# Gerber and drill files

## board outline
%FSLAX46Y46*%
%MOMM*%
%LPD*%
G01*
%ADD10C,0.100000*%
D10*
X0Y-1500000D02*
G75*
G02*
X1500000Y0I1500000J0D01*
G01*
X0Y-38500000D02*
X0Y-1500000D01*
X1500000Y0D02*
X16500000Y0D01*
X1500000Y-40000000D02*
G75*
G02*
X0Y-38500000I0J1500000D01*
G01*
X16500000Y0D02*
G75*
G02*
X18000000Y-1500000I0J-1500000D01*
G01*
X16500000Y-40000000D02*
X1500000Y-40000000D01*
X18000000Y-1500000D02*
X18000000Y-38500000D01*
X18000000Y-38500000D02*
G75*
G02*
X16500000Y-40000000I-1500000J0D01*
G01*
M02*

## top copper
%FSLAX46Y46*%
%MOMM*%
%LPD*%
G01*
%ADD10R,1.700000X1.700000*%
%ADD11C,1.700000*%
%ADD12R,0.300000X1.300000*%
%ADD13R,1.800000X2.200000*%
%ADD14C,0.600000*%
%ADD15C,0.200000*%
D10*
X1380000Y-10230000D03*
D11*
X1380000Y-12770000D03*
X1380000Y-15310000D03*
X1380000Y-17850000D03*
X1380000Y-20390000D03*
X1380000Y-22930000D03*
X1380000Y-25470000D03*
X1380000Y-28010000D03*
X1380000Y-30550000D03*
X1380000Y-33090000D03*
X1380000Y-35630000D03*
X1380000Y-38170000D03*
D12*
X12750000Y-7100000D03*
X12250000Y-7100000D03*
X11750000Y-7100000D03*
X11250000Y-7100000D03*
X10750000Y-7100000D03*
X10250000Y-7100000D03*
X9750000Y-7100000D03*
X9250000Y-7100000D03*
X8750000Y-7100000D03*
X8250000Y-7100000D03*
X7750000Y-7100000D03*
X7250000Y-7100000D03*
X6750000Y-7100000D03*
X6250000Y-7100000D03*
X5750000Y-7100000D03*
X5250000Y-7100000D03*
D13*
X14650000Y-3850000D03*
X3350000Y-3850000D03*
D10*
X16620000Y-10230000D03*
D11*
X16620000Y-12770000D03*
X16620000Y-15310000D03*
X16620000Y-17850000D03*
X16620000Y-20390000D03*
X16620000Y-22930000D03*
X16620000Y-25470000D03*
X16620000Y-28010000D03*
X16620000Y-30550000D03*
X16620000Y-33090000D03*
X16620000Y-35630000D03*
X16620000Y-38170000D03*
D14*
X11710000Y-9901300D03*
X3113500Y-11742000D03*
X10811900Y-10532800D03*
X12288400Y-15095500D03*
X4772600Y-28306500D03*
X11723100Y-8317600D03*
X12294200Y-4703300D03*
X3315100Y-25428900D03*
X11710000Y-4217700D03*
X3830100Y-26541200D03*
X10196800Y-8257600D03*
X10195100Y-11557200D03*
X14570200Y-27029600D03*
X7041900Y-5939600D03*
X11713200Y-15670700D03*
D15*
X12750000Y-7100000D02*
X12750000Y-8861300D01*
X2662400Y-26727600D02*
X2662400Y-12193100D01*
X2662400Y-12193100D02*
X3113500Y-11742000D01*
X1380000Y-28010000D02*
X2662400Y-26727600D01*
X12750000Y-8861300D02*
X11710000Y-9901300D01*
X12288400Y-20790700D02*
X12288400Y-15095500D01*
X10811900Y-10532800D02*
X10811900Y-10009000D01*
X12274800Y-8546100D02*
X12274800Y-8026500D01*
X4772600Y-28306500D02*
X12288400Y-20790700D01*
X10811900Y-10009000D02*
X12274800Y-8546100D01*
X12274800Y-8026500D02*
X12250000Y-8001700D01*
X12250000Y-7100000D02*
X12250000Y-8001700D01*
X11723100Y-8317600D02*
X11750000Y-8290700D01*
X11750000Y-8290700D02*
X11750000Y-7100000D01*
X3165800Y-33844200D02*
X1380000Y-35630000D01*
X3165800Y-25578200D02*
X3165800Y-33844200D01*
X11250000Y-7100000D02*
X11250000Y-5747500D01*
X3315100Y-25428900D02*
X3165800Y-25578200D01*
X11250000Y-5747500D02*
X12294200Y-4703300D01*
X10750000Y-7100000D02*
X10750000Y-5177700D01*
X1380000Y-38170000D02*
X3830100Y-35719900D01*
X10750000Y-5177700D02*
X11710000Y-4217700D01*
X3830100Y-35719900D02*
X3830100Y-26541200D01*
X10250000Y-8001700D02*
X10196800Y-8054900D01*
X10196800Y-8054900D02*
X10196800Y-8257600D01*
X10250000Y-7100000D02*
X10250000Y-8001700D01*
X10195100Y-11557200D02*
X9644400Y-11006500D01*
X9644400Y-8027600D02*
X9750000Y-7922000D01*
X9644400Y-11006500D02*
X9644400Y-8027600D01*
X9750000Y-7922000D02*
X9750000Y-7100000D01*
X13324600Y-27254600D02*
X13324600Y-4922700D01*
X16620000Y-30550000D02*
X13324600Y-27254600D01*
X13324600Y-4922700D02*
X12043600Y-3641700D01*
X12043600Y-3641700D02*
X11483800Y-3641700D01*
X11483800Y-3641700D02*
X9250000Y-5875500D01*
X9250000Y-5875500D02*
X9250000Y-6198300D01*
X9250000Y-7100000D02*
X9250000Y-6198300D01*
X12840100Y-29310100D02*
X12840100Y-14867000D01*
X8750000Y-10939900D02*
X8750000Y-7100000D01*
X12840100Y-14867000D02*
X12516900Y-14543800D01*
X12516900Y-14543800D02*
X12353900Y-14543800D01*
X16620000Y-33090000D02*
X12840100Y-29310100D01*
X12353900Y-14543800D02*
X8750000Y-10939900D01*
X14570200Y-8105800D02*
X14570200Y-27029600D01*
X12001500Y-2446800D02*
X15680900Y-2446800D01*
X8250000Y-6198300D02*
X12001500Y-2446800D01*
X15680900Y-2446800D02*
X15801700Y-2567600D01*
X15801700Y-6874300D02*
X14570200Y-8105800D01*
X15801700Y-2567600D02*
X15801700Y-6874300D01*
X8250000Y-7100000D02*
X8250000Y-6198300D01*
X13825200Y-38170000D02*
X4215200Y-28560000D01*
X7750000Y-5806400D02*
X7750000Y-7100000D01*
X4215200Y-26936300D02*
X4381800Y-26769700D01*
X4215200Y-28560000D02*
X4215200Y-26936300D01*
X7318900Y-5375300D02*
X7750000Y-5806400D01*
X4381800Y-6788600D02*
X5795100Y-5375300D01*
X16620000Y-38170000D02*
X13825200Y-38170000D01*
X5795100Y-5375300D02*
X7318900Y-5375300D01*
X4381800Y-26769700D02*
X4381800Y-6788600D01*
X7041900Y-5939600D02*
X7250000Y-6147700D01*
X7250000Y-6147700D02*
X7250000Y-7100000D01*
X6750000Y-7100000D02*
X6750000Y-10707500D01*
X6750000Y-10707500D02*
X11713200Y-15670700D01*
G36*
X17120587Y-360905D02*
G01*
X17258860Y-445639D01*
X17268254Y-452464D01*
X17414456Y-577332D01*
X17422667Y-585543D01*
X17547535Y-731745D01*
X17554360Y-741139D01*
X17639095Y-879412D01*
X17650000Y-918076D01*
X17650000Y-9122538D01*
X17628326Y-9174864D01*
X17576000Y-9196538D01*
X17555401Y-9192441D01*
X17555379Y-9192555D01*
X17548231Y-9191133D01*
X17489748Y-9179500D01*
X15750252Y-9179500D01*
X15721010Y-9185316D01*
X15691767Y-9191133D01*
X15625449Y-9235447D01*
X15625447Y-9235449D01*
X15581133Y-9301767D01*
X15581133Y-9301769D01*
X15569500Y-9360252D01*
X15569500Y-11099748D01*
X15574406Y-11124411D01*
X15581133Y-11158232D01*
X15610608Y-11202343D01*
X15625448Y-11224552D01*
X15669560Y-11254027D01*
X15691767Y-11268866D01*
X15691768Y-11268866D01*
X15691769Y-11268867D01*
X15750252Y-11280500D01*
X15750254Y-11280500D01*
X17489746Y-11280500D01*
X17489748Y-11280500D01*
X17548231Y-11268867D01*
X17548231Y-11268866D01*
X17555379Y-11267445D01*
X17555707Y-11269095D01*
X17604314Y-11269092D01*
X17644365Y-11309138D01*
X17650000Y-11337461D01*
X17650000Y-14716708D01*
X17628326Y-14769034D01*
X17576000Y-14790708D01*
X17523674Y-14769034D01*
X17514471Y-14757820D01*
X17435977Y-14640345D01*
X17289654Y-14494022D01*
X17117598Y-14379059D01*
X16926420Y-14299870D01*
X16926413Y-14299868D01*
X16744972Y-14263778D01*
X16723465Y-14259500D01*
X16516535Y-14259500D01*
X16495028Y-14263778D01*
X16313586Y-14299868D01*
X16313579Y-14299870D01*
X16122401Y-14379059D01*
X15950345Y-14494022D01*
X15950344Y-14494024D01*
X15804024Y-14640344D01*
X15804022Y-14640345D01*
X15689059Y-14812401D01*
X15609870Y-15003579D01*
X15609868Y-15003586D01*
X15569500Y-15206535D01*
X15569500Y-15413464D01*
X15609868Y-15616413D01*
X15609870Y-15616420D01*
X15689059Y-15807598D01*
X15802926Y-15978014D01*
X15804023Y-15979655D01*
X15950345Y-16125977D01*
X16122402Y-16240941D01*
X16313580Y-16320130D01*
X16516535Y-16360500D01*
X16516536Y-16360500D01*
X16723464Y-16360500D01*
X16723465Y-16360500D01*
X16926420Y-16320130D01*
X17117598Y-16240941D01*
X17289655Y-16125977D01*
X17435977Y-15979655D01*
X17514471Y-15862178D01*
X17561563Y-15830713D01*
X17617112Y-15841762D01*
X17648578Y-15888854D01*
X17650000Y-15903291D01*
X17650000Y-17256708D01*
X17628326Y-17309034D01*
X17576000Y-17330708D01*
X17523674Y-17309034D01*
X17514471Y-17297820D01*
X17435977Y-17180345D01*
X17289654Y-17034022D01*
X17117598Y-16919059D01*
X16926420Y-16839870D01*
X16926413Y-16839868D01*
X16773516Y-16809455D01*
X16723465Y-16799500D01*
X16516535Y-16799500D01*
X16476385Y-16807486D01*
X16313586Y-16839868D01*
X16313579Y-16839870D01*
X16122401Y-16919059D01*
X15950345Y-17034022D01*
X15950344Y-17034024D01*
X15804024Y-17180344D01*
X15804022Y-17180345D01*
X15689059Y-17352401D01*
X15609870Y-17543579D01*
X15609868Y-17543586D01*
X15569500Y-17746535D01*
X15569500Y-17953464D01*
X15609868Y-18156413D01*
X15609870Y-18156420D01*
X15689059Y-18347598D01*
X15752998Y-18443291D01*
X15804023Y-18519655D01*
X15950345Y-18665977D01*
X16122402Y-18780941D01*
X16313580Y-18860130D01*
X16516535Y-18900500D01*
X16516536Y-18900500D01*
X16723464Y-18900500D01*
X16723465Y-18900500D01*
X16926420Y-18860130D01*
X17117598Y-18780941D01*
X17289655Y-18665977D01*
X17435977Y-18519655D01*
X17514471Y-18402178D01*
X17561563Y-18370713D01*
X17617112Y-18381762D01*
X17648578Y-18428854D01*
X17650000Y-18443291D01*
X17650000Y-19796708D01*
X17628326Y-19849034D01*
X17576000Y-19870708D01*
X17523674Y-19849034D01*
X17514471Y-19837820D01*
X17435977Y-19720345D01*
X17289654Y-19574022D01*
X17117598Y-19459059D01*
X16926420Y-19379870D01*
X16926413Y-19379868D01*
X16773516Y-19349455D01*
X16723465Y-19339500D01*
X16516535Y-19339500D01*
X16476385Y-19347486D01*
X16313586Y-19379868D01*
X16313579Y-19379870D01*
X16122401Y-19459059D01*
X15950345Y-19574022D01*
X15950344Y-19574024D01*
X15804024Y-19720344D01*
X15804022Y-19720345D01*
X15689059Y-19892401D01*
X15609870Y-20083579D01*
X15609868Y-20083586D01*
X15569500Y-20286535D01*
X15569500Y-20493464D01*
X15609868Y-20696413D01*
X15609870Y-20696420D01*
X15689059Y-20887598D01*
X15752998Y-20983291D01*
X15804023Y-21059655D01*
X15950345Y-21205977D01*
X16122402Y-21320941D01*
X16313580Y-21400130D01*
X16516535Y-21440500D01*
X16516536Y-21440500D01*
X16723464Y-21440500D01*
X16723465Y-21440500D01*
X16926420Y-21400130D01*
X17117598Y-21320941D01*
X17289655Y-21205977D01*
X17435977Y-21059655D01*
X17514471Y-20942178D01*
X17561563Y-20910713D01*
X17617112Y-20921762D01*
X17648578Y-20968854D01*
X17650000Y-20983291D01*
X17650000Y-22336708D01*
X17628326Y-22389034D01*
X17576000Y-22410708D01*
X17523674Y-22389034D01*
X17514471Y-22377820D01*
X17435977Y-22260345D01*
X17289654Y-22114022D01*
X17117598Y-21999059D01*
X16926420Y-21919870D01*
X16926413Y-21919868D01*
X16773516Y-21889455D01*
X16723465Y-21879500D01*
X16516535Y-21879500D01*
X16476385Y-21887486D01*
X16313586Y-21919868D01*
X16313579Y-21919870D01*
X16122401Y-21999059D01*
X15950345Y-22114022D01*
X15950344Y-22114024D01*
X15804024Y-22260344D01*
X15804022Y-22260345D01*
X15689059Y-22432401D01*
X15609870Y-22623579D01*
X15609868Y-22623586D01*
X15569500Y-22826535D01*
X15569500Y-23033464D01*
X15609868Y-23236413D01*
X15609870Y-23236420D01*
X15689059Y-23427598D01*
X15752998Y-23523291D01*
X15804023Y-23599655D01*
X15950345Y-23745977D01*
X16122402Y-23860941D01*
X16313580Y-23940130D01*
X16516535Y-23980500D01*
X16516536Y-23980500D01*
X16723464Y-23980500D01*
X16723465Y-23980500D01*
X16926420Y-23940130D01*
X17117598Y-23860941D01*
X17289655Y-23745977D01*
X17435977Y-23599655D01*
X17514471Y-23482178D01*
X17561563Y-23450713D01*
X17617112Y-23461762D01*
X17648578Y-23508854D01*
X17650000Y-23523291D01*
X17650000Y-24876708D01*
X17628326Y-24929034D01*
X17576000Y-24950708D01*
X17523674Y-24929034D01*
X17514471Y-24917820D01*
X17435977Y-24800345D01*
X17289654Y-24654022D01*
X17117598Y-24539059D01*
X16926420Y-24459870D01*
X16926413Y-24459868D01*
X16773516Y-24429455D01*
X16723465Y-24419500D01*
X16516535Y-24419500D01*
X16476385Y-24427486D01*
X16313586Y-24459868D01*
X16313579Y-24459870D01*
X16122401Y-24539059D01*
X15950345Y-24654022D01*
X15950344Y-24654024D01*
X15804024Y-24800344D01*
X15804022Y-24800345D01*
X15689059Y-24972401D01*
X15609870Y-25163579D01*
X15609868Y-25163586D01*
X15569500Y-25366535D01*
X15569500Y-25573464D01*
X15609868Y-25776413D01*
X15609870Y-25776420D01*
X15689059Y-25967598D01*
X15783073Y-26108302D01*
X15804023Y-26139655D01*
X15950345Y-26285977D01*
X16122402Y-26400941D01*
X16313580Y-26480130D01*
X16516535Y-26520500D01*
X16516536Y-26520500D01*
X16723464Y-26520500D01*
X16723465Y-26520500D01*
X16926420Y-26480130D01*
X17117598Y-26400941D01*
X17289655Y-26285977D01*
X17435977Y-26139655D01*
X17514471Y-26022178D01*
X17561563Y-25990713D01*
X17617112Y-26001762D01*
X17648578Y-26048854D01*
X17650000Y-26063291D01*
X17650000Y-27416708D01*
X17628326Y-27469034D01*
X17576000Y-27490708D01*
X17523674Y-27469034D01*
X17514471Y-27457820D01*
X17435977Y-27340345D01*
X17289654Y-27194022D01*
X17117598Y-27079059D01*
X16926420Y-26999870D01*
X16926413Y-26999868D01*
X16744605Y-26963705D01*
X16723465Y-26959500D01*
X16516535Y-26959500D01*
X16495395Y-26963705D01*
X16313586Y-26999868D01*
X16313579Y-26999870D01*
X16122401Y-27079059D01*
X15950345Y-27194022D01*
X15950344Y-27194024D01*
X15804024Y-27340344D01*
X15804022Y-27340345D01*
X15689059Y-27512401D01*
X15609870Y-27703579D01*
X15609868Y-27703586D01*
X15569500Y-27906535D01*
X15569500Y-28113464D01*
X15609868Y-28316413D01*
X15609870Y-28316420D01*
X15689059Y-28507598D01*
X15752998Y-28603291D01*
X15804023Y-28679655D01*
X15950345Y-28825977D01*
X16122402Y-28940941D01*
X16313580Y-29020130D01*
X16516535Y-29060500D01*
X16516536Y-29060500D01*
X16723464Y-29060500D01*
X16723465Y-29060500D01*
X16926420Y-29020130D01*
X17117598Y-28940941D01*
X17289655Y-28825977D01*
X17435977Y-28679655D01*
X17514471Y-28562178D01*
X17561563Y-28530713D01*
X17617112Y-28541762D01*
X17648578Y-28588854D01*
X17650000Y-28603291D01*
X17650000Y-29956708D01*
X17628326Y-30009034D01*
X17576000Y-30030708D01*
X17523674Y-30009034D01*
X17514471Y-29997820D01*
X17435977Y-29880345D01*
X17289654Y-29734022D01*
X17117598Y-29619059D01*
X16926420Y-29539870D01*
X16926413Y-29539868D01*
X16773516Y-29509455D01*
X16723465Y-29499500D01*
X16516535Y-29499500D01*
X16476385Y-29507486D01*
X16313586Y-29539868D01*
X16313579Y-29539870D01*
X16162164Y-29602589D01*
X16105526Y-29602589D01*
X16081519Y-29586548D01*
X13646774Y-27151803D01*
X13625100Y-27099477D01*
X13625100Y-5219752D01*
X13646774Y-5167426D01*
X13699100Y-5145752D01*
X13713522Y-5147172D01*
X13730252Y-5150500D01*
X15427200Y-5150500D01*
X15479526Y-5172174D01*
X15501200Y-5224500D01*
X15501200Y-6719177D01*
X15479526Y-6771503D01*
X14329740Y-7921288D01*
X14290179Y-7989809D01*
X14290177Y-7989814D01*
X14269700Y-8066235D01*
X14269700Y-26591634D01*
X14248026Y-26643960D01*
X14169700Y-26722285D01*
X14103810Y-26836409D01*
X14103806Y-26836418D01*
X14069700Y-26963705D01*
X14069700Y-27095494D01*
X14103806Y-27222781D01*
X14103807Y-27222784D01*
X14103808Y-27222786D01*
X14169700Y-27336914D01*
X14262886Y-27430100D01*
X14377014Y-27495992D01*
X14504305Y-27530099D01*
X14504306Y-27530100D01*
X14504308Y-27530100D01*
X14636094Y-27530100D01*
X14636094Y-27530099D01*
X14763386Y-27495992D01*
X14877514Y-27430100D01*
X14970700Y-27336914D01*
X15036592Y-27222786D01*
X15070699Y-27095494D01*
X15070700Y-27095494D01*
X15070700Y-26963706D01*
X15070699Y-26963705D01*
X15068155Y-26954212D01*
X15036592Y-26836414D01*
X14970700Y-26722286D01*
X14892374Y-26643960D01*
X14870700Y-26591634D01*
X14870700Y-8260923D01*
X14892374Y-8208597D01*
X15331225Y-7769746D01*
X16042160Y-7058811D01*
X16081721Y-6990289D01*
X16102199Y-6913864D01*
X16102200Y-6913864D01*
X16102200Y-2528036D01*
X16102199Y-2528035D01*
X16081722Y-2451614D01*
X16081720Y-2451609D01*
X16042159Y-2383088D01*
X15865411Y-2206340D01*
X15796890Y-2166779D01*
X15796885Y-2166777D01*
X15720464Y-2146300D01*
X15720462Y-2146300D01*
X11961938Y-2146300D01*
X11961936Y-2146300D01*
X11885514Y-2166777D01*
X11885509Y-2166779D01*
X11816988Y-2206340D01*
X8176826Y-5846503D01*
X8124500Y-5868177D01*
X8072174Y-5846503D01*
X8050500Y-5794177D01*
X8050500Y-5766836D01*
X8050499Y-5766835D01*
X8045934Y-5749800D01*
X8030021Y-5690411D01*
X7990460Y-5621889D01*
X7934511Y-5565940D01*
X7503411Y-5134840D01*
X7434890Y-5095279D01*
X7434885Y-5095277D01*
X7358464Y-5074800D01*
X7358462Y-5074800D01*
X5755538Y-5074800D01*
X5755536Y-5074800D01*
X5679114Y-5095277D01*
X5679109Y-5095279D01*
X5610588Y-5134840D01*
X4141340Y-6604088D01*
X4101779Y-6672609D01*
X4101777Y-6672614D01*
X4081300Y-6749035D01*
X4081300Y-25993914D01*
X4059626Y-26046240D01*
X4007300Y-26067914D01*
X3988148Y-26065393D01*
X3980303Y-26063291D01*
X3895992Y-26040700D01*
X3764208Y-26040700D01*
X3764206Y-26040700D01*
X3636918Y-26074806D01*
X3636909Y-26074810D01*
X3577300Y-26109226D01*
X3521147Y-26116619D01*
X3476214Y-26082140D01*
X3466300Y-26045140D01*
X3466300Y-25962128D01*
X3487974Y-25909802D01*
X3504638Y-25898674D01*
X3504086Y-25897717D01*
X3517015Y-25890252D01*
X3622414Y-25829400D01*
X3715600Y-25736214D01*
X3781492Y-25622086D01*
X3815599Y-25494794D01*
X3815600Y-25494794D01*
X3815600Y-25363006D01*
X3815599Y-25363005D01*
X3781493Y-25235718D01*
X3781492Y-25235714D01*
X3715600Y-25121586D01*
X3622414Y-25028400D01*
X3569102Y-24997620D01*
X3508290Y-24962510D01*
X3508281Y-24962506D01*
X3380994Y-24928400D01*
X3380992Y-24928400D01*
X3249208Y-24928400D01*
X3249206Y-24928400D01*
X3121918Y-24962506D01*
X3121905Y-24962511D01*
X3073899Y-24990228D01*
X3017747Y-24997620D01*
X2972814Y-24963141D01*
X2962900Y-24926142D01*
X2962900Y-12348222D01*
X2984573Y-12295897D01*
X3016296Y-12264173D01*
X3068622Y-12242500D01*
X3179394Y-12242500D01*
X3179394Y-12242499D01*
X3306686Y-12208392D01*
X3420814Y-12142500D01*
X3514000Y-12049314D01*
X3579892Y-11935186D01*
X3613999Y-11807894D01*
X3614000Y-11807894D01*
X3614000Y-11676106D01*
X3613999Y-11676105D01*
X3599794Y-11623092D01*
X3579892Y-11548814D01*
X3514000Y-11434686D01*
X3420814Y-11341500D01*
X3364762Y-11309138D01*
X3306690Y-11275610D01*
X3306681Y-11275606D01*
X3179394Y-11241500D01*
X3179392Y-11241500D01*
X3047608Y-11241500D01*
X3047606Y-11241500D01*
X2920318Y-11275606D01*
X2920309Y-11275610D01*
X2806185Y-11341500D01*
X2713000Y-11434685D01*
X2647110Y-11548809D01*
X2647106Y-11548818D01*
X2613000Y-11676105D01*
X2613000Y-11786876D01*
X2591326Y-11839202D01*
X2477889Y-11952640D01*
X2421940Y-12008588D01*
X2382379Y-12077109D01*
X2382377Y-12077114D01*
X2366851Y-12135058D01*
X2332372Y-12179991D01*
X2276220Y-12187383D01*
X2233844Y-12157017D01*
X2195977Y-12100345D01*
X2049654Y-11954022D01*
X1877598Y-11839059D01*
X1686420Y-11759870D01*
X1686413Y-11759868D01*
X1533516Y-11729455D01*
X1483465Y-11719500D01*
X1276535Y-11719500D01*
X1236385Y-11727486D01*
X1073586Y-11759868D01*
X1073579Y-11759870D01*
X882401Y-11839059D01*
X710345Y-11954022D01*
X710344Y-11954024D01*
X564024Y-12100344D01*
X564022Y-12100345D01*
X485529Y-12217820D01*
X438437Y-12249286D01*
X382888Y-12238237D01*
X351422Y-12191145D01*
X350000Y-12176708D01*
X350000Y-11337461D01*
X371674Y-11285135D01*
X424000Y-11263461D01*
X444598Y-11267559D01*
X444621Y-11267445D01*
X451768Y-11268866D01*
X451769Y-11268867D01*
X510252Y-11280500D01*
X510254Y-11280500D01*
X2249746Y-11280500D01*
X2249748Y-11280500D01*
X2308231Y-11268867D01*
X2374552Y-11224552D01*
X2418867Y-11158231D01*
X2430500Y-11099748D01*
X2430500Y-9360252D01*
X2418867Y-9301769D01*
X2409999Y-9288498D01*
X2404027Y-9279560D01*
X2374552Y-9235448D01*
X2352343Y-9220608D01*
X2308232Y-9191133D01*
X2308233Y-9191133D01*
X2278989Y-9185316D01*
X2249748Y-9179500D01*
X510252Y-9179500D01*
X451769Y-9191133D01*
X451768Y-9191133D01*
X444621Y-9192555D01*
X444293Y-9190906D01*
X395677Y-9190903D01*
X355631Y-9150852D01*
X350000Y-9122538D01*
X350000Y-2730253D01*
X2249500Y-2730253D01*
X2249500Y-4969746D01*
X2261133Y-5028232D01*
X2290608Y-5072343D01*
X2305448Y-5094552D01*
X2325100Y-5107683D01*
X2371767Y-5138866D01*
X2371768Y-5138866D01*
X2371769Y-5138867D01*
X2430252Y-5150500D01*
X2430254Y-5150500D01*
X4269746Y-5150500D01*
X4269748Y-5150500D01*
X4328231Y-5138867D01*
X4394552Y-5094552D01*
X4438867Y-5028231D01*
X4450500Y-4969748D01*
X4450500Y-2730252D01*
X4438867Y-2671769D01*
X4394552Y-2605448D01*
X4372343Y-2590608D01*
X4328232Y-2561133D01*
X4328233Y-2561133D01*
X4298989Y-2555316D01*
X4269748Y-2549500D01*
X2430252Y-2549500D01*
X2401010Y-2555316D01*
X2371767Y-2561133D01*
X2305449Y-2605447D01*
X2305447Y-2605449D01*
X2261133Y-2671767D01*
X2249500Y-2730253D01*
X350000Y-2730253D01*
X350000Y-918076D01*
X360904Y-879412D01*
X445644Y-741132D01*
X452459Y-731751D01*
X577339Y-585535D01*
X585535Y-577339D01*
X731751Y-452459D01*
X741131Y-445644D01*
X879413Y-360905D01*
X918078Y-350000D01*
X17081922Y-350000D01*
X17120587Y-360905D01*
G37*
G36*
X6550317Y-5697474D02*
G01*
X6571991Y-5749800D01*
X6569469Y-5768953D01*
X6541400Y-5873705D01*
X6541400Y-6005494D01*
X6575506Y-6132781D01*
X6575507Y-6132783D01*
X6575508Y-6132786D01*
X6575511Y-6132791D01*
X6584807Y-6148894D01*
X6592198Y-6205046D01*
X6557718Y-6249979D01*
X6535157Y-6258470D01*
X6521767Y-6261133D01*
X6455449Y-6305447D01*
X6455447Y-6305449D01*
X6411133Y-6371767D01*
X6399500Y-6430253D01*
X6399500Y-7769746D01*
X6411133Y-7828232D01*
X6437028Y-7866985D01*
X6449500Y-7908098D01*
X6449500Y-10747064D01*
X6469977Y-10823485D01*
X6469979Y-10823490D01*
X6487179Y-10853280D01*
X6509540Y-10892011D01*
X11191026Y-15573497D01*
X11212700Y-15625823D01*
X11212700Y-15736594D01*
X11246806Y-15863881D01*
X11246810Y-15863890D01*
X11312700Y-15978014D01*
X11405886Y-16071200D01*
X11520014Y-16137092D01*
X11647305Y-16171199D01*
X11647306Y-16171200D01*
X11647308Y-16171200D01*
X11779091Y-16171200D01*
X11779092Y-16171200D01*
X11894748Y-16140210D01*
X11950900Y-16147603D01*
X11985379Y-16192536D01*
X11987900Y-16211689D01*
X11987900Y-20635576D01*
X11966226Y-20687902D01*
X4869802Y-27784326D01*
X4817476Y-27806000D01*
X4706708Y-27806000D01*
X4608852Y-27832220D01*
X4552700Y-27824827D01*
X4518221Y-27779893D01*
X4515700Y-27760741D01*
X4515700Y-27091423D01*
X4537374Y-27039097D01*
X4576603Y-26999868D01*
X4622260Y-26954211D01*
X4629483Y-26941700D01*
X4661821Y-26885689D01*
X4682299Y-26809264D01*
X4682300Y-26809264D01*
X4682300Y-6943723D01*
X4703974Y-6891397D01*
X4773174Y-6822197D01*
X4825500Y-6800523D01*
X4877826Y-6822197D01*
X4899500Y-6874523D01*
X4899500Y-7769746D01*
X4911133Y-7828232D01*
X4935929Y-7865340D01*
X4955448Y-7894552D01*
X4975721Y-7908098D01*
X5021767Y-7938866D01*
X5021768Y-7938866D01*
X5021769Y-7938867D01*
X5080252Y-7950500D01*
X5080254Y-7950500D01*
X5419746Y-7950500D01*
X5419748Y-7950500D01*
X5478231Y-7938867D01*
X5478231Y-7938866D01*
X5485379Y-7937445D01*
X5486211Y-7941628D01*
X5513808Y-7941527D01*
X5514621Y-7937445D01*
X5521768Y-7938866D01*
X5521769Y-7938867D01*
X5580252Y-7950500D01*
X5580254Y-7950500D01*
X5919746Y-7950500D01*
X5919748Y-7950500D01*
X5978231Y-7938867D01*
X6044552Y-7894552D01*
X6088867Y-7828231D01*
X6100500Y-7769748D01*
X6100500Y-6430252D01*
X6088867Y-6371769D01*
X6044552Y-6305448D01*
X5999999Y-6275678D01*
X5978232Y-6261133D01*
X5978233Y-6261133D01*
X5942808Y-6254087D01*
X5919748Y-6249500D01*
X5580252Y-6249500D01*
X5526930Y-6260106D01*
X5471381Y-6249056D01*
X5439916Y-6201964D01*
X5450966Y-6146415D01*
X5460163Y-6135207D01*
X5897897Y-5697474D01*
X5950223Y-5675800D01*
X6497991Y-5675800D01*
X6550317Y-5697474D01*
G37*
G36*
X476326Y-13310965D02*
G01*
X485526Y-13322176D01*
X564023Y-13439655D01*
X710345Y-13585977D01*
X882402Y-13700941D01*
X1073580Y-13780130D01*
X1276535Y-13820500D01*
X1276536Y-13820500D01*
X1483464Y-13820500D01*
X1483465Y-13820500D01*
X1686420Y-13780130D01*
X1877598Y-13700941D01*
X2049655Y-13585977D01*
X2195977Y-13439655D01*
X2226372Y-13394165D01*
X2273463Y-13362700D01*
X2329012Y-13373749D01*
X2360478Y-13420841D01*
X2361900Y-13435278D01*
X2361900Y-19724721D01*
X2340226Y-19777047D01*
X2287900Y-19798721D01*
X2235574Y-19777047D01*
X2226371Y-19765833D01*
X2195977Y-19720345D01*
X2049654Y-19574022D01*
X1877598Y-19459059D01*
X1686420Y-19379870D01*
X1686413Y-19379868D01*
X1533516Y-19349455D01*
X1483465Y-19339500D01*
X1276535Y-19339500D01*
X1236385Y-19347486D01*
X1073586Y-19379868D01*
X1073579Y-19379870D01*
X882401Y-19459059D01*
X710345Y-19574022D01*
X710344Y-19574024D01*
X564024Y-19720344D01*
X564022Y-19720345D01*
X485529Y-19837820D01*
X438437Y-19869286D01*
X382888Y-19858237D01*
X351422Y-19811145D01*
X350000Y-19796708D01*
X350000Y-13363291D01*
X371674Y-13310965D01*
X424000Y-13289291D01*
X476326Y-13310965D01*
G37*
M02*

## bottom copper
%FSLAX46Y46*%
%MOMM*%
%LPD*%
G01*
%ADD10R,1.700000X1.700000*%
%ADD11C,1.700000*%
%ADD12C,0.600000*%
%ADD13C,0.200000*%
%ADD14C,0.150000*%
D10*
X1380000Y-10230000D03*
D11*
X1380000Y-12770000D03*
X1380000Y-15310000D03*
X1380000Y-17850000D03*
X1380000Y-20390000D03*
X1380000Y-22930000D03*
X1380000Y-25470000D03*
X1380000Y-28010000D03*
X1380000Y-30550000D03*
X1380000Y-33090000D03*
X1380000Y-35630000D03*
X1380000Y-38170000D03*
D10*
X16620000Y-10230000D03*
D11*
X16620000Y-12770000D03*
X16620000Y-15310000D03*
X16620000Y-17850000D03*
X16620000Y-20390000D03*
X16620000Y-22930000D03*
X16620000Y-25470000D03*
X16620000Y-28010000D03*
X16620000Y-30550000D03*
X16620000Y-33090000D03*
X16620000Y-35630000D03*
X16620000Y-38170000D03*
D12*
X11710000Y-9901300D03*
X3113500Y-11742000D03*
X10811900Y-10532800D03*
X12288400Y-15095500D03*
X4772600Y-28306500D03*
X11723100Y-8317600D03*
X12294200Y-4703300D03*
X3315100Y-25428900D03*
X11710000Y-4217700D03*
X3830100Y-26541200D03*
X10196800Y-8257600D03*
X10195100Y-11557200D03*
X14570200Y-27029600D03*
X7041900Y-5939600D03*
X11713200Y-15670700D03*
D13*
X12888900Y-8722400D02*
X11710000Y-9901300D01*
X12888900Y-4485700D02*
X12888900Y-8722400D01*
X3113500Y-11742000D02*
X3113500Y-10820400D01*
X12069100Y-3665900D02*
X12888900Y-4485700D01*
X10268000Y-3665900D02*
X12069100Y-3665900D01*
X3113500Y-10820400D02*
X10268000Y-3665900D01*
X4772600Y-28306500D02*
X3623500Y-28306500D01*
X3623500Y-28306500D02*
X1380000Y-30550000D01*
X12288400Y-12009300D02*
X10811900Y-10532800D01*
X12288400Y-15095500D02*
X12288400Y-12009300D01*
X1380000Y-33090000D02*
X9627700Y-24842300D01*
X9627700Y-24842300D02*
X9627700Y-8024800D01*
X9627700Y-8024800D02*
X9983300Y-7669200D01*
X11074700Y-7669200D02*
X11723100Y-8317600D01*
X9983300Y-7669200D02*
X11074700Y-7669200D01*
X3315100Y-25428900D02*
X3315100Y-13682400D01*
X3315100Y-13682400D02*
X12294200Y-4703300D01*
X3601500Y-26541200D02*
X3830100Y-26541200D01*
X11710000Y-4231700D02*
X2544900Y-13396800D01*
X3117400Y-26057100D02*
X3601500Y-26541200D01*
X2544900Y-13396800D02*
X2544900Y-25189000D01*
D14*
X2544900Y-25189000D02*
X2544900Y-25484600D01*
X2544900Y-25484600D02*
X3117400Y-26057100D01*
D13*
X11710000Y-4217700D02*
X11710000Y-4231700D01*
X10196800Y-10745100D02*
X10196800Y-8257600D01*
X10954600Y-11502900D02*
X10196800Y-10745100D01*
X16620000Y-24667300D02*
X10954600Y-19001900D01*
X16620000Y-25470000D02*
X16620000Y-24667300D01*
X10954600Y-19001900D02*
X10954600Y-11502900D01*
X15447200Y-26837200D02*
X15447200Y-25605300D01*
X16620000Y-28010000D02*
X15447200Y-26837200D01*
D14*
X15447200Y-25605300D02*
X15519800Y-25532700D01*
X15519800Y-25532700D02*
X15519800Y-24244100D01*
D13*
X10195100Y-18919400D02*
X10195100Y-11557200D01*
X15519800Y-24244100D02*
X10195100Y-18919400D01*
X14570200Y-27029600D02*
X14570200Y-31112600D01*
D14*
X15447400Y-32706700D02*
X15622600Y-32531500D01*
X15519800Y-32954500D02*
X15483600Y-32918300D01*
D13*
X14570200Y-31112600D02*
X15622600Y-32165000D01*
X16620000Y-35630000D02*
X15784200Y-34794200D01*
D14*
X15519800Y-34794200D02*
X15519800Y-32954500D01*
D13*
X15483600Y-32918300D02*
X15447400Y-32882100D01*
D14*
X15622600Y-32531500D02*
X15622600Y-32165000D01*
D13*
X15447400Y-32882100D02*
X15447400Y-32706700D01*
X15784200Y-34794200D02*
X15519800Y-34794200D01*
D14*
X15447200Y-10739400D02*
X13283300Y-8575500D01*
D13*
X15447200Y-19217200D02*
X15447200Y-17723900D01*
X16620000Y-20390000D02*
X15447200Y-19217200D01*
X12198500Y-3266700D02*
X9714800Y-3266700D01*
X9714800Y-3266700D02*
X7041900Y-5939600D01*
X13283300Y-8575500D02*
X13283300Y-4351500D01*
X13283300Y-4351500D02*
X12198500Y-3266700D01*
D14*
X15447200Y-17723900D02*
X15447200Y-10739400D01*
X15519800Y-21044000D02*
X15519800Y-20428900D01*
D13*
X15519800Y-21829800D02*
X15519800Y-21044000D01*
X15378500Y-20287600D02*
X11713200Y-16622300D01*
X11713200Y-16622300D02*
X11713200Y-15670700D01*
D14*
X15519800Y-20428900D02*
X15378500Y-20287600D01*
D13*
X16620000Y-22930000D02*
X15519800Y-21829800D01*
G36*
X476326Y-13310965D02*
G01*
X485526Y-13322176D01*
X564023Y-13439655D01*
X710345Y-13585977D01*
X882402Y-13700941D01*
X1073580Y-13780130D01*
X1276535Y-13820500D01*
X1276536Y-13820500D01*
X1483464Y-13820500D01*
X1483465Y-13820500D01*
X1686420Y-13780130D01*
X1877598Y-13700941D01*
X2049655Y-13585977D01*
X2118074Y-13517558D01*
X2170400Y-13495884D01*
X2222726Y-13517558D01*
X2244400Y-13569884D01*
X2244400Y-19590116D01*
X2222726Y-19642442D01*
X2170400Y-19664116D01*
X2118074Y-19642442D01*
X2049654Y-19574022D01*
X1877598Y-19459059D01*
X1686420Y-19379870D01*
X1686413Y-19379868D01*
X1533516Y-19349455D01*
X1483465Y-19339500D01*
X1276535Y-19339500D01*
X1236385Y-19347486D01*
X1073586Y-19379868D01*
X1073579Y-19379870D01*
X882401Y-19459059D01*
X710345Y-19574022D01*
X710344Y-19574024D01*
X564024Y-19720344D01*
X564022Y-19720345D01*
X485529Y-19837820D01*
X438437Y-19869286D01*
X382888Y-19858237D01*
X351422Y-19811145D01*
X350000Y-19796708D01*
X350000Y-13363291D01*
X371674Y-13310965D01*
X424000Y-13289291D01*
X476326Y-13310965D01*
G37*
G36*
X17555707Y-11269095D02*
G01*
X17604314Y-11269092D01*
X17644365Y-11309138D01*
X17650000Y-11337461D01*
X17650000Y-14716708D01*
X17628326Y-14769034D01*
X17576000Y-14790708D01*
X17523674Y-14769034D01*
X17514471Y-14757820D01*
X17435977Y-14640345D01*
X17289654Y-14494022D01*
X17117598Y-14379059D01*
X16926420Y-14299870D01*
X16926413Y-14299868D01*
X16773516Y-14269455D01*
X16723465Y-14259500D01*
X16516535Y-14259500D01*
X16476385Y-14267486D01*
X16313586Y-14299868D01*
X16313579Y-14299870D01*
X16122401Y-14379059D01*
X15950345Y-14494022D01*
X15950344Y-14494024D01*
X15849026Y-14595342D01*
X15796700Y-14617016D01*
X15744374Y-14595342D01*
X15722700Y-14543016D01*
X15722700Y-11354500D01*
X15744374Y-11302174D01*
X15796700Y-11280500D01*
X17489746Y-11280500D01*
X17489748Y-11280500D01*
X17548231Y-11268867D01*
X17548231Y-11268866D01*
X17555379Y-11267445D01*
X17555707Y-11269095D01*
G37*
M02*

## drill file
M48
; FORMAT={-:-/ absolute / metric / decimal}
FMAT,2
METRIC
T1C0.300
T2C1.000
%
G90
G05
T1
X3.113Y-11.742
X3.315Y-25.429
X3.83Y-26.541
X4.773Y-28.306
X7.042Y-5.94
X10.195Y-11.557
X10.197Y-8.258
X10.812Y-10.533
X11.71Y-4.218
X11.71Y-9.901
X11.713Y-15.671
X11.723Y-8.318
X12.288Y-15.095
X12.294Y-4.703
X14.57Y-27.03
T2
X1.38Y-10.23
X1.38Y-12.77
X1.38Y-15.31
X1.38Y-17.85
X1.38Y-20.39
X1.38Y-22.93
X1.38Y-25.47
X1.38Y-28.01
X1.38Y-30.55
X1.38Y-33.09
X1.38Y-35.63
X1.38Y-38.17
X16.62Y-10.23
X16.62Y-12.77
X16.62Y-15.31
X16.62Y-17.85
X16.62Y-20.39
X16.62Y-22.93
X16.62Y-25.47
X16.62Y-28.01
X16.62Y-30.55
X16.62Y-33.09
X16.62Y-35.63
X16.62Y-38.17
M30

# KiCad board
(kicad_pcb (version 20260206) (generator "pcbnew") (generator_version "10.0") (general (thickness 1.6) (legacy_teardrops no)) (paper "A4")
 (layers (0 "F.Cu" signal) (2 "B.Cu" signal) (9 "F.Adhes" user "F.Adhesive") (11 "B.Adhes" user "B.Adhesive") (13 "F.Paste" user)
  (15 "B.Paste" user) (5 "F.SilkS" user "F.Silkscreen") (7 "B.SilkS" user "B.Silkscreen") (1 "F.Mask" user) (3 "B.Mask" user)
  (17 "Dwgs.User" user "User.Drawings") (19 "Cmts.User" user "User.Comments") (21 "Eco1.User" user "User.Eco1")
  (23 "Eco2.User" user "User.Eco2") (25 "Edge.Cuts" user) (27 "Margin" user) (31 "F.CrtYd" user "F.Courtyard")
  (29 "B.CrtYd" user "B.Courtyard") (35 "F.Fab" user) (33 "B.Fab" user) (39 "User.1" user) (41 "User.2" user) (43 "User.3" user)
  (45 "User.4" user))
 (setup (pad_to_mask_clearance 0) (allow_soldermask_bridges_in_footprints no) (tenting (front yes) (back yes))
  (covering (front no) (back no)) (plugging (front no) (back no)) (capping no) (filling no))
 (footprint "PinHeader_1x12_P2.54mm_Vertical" (layer "F.Cu") (at 1.38 10.23)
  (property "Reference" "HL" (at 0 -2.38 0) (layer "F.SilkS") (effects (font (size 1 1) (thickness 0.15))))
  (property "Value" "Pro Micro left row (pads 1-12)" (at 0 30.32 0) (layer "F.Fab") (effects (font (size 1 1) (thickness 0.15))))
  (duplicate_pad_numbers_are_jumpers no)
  (pad "1" thru_hole rect (at 0 0) (size 1.7 1.7) (drill 1) (layers "*.Cu" "*.Mask") (remove_unused_layers no))
  (pad "2" thru_hole circle (at 0 2.54) (size 1.7 1.7) (drill 1) (layers "*.Cu" "*.Mask") (remove_unused_layers no))
  (pad "3" thru_hole circle (at 0 5.08) (size 1.7 1.7) (drill 1) (layers "*.Cu" "*.Mask") (remove_unused_layers no) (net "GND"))
  (pad "4" thru_hole circle (at 0 7.62) (size 1.7 1.7) (drill 1) (layers "*.Cu" "*.Mask") (remove_unused_layers no) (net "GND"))
  (pad "5" thru_hole circle (at 0 10.16) (size 1.7 1.7) (drill 1) (layers "*.Cu" "*.Mask") (remove_unused_layers no))
  (pad "6" thru_hole circle (at 0 12.7) (size 1.7 1.7) (drill 1) (layers "*.Cu" "*.Mask") (remove_unused_layers no))
  (pad "7" thru_hole circle (at 0 15.24) (size 1.7 1.7) (drill 1) (layers "*.Cu" "*.Mask") (remove_unused_layers no))
  (pad "8" thru_hole circle (at 0 17.78) (size 1.7 1.7) (drill 1) (layers "*.Cu" "*.Mask") (remove_unused_layers no) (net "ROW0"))
  (pad "9" thru_hole circle (at 0 20.32) (size 1.7 1.7) (drill 1) (layers "*.Cu" "*.Mask") (remove_unused_layers no) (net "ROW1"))
  (pad "10" thru_hole circle (at 0 22.86) (size 1.7 1.7) (drill 1) (layers "*.Cu" "*.Mask") (remove_unused_layers no) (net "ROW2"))
  (pad "11" thru_hole circle (at 0 25.4) (size 1.7 1.7) (drill 1) (layers "*.Cu" "*.Mask") (remove_unused_layers no) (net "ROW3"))
  (pad "12" thru_hole circle (at 0 27.94) (size 1.7 1.7) (drill 1) (layers "*.Cu" "*.Mask") (remove_unused_layers no) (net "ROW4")))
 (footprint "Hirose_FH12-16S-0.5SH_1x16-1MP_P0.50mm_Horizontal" (layer "F.Cu") (at 9 5.25 180)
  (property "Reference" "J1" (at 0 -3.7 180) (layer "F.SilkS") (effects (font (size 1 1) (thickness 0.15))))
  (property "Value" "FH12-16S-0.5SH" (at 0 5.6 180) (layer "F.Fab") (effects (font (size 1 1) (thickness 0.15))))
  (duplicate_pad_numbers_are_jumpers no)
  (pad "1" smd rect (at -3.75 -1.85 180) (size 0.3 1.3) (layers "F.Cu" "F.Mask" "F.Paste") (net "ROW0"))
  (pad "2" smd rect (at -3.25 -1.85 180) (size 0.3 1.3) (layers "F.Cu" "F.Mask" "F.Paste") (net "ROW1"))
  (pad "3" smd rect (at -2.75 -1.85 180) (size 0.3 1.3) (layers "F.Cu" "F.Mask" "F.Paste") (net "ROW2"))
  (pad "4" smd rect (at -2.25 -1.85 180) (size 0.3 1.3) (layers "F.Cu" "F.Mask" "F.Paste") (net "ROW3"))
  (pad "5" smd rect (at -1.75 -1.85 180) (size 0.3 1.3) (layers "F.Cu" "F.Mask" "F.Paste") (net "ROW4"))
  (pad "6" smd rect (at -1.25 -1.85 180) (size 0.3 1.3) (layers "F.Cu" "F.Mask" "F.Paste") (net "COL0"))
  (pad "7" smd rect (at -0.75 -1.85 180) (size 0.3 1.3) (layers "F.Cu" "F.Mask" "F.Paste") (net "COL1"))
  (pad "8" smd rect (at -0.25 -1.85 180) (size 0.3 1.3) (layers "F.Cu" "F.Mask" "F.Paste") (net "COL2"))
  (pad "9" smd rect (at 0.25 -1.85 180) (size 0.3 1.3) (layers "F.Cu" "F.Mask" "F.Paste") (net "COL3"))
  (pad "10" smd rect (at 0.75 -1.85 180) (size 0.3 1.3) (layers "F.Cu" "F.Mask" "F.Paste") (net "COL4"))
  (pad "11" smd rect (at 1.25 -1.85 180) (size 0.3 1.3) (layers "F.Cu" "F.Mask" "F.Paste") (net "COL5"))
  (pad "12" smd rect (at 1.75 -1.85 180) (size 0.3 1.3) (layers "F.Cu" "F.Mask" "F.Paste") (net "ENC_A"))
  (pad "13" smd rect (at 2.25 -1.85 180) (size 0.3 1.3) (layers "F.Cu" "F.Mask" "F.Paste") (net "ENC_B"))
  (pad "14" smd rect (at 2.75 -1.85 180) (size 0.3 1.3) (layers "F.Cu" "F.Mask" "F.Paste") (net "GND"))
  (pad "15" smd rect (at 3.25 -1.85 180) (size 0.3 1.3) (layers "F.Cu" "F.Mask" "F.Paste"))
  (pad "16" smd rect (at 3.75 -1.85 180) (size 0.3 1.3) (layers "F.Cu" "F.Mask" "F.Paste"))
  (pad "MP" smd rect (at -5.65 1.4 180) (size 1.8 2.2) (layers "F.Cu" "F.Mask" "F.Paste"))
  (pad "MP" smd rect (at 5.65 1.4 180) (size 1.8 2.2) (layers "F.Cu" "F.Mask" "F.Paste")))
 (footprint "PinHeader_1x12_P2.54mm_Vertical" (layer "F.Cu") (at 16.62 10.23)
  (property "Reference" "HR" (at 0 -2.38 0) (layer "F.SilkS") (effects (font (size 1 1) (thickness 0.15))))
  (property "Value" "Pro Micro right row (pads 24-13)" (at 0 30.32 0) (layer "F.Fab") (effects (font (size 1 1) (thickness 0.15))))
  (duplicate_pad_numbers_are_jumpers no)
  (pad "1" thru_hole rect (at 0 0) (size 1.7 1.7) (drill 1) (layers "*.Cu" "*.Mask") (remove_unused_layers no))
  (pad "2" thru_hole circle (at 0 2.54) (size 1.7 1.7) (drill 1) (layers "*.Cu" "*.Mask") (remove_unused_layers no) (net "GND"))
  (pad "3" thru_hole circle (at 0 5.08) (size 1.7 1.7) (drill 1) (layers "*.Cu" "*.Mask") (remove_unused_layers no))
  (pad "4" thru_hole circle (at 0 7.62) (size 1.7 1.7) (drill 1) (layers "*.Cu" "*.Mask") (remove_unused_layers no))
  (pad "5" thru_hole circle (at 0 10.16) (size 1.7 1.7) (drill 1) (layers "*.Cu" "*.Mask") (remove_unused_layers no) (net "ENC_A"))
  (pad "6" thru_hole circle (at 0 12.7) (size 1.7 1.7) (drill 1) (layers "*.Cu" "*.Mask") (remove_unused_layers no) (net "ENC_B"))
  (pad "7" thru_hole circle (at 0 15.24) (size 1.7 1.7) (drill 1) (layers "*.Cu" "*.Mask") (remove_unused_layers no) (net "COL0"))
  (pad "8" thru_hole circle (at 0 17.78) (size 1.7 1.7) (drill 1) (layers "*.Cu" "*.Mask") (remove_unused_layers no) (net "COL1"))
  (pad "9" thru_hole circle (at 0 20.32) (size 1.7 1.7) (drill 1) (layers "*.Cu" "*.Mask") (remove_unused_layers no) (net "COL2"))
  (pad "10" thru_hole circle (at 0 22.86) (size 1.7 1.7) (drill 1) (layers "*.Cu" "*.Mask") (remove_unused_layers no) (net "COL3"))
  (pad "11" thru_hole circle (at 0 25.4) (size 1.7 1.7) (drill 1) (layers "*.Cu" "*.Mask") (remove_unused_layers no) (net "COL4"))
  (pad "12" thru_hole circle (at 0 27.94) (size 1.7 1.7) (drill 1) (layers "*.Cu" "*.Mask") (remove_unused_layers no) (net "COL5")))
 (gr_arc (start 0 1.5) (mid 0.43934 0.43934) (end 1.5 0) (stroke (width 0.1) (type default)) (layer "Edge.Cuts"))
 (gr_line (start 0 38.5) (end 0 1.5) (stroke (width 0.1) (type default)) (layer "Edge.Cuts"))
 (gr_line (start 1.5 0) (end 16.5 0) (stroke (width 0.1) (type default)) (layer "Edge.Cuts"))
 (gr_arc (start 1.5 40) (mid 0.43934 39.56066) (end 0 38.5) (stroke (width 0.1) (type default)) (layer "Edge.Cuts"))
 (gr_arc (start 16.5 0) (mid 17.56066 0.43934) (end 18 1.5) (stroke (width 0.1) (type default)) (layer "Edge.Cuts"))
 (gr_line (start 16.5 40) (end 1.5 40) (stroke (width 0.1) (type default)) (layer "Edge.Cuts"))
 (gr_line (start 18 1.5) (end 18 38.5) (stroke (width 0.1) (type default)) (layer "Edge.Cuts"))
 (gr_arc (start 18 38.5) (mid 17.56066 39.56066) (end 16.5 40) (stroke (width 0.1) (type default)) (layer "Edge.Cuts"))
 (segment (start 12.75 7.1) (end 12.75 8.8613) (width 0.2) (layer "F.Cu") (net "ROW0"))
 (segment (start 2.6624 26.7276) (end 2.6624 12.1931) (width 0.2) (layer "F.Cu") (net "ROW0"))
 (segment (start 2.6624 12.1931) (end 3.1135 11.742) (width 0.2) (layer "F.Cu") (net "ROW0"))
 (segment (start 1.38 28.01) (end 2.6624 26.7276) (width 0.2) (layer "F.Cu") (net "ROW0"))
 (segment (start 12.75 8.8613) (end 11.71 9.9013) (width 0.2) (layer "F.Cu") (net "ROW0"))
 (via (at 11.71 9.9013) (size 0.6) (drill 0.3) (layers "F.Cu" "B.Cu") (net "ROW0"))
 (via (at 3.1135 11.742) (size 0.6) (drill 0.3) (layers "F.Cu" "B.Cu") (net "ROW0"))
 (segment (start 12.8889 8.7224) (end 11.71 9.9013) (width 0.2) (layer "B.Cu") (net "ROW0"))
 (segment (start 12.8889 4.4857) (end 12.8889 8.7224) (width 0.2) (layer "B.Cu") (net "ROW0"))
 (segment (start 3.1135 11.742) (end 3.1135 10.8204) (width 0.2) (layer "B.Cu") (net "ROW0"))
 (segment (start 12.0691 3.6659) (end 12.8889 4.4857) (width 0.2) (layer "B.Cu") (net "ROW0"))
 (segment (start 10.268 3.6659) (end 12.0691 3.6659) (width 0.2) (layer "B.Cu") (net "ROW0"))
 (segment (start 3.1135 10.8204) (end 10.268 3.6659) (width 0.2) (layer "B.Cu") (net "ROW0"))
 (segment (start 12.2884 20.7907) (end 12.2884 15.0955) (width 0.2) (layer "F.Cu") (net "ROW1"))
 (segment (start 10.8119 10.5328) (end 10.8119 10.009) (width 0.2) (layer "F.Cu") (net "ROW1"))
 (segment (start 12.2748 8.5461) (end 12.2748 8.0265) (width 0.2) (layer "F.Cu") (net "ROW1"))
 (segment (start 4.7726 28.3065) (end 12.2884 20.7907) (width 0.2) (layer "F.Cu") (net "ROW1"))
 (segment (start 10.8119 10.009) (end 12.2748 8.5461) (width 0.2) (layer "F.Cu") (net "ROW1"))
 (segment (start 12.2748 8.0265) (end 12.25 8.0017) (width 0.2) (layer "F.Cu") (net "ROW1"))
 (segment (start 12.25 7.1) (end 12.25 8.0017) (width 0.2) (layer "F.Cu") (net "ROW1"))
 (via (at 10.8119 10.5328) (size 0.6) (drill 0.3) (layers "F.Cu" "B.Cu") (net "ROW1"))
 (via (at 12.2884 15.0955) (size 0.6) (drill 0.3) (layers "F.Cu" "B.Cu") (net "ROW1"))
 (via (at 4.7726 28.3065) (size 0.6) (drill 0.3) (layers "F.Cu" "B.Cu") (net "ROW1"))
 (segment (start 4.7726 28.3065) (end 3.6235 28.3065) (width 0.2) (layer "B.Cu") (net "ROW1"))
 (segment (start 3.6235 28.3065) (end 1.38 30.55) (width 0.2) (layer "B.Cu") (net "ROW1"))
 (segment (start 12.2884 12.0093) (end 10.8119 10.5328) (width 0.2) (layer "B.Cu") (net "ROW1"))
 (segment (start 12.2884 15.0955) (end 12.2884 12.0093) (width 0.2) (layer "B.Cu") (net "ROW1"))
 (segment (start 11.7231 8.3176) (end 11.75 8.2907) (width 0.2) (layer "F.Cu") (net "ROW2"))
 (segment (start 11.75 8.2907) (end 11.75 7.1) (width 0.2) (layer "F.Cu") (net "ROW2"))
 (via (at 11.7231 8.3176) (size 0.6) (drill 0.3) (layers "F.Cu" "B.Cu") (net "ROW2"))
 (segment (start 1.38 33.09) (end 9.6277 24.8423) (width 0.2) (layer "B.Cu") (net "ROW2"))
 (segment (start 9.6277 24.8423) (end 9.6277 8.0248) (width 0.2) (layer "B.Cu") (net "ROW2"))
 (segment (start 9.6277 8.0248) (end 9.9833 7.6692) (width 0.2) (layer "B.Cu") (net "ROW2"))
 (segment (start 11.0747 7.6692) (end 11.7231 8.3176) (width 0.2) (layer "B.Cu") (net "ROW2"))
 (segment (start 9.9833 7.6692) (end 11.0747 7.6692) (width 0.2) (layer "B.Cu") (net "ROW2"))
 (segment (start 3.1658 33.8442) (end 1.38 35.63) (width 0.2) (layer "F.Cu") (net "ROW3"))
 (segment (start 3.1658 25.5782) (end 3.1658 33.8442) (width 0.2) (layer "F.Cu") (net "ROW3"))
 (segment (start 11.25 7.1) (end 11.25 5.7475) (width 0.2) (layer "F.Cu") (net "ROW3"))
 (segment (start 3.3151 25.4289) (end 3.1658 25.5782) (width 0.2) (layer "F.Cu") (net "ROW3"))
 (segment (start 11.25 5.7475) (end 12.2942 4.7033) (width 0.2) (layer "F.Cu") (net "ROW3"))
 (via (at 12.2942 4.7033) (size 0.6) (drill 0.3) (layers "F.Cu" "B.Cu") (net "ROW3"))
 (via (at 3.3151 25.4289) (size 0.6) (drill 0.3) (layers "F.Cu" "B.Cu") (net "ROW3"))
 (segment (start 3.3151 25.4289) (end 3.3151 13.6824) (width 0.2) (layer "B.Cu") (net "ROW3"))
 (segment (start 3.3151 13.6824) (end 12.2942 4.7033) (width 0.2) (layer "B.Cu") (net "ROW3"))
 (segment (start 10.75 7.1) (end 10.75 5.1777) (width 0.2) (layer "F.Cu") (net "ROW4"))
 (segment (start 1.38 38.17) (end 3.8301 35.7199) (width 0.2) (layer "F.Cu") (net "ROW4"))
 (segment (start 10.75 5.1777) (end 11.71 4.2177) (width 0.2) (layer "F.Cu") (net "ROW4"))
 (segment (start 3.8301 35.7199) (end 3.8301 26.5412) (width 0.2) (layer "F.Cu") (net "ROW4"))
 (via (at 11.71 4.2177) (size 0.6) (drill 0.3) (layers "F.Cu" "B.Cu") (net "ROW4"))
 (via (at 3.8301 26.5412) (size 0.6) (drill 0.3) (layers "F.Cu" "B.Cu") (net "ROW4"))
 (segment (start 3.6015 26.5412) (end 3.8301 26.5412) (width 0.2) (layer "B.Cu") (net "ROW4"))
 (segment (start 11.71 4.2317) (end 2.5449 13.3968) (width 0.2) (layer "B.Cu") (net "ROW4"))
 (segment (start 3.1174 26.0571) (end 3.6015 26.5412) (width 0.2) (layer "B.Cu") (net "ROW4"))
 (segment (start 2.5449 13.3968) (end 2.5449 25.189) (width 0.2) (layer "B.Cu") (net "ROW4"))
 (segment (start 2.5449 25.189) (end 2.5449 25.4846) (width 0.15) (layer "B.Cu") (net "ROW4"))
 (segment (start 2.5449 25.4846) (end 3.1174 26.0571) (width 0.15) (layer "B.Cu") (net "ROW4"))
 (segment (start 11.71 4.2177) (end 11.71 4.2317) (width 0.2) (layer "B.Cu") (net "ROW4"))
 (segment (start 10.25 8.0017) (end 10.1968 8.0549) (width 0.2) (layer "F.Cu") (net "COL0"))
 (segment (start 10.1968 8.0549) (end 10.1968 8.2576) (width 0.2) (layer "F.Cu") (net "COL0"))
 (segment (start 10.25 7.1) (end 10.25 8.0017) (width 0.2) (layer "F.Cu") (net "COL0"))
 (via (at 10.1968 8.2576) (size 0.6) (drill 0.3) (layers "F.Cu" "B.Cu") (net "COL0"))
 (segment (start 10.1968 10.7451) (end 10.1968 8.2576) (width 0.2) (layer "B.Cu") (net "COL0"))
 (segment (start 10.9546 11.5029) (end 10.1968 10.7451) (width 0.2) (layer "B.Cu") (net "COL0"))
 (segment (start 16.62 24.6673) (end 10.9546 19.0019) (width 0.2) (layer "B.Cu") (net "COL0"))
 (segment (start 16.62 25.47) (end 16.62 24.6673) (width 0.2) (layer "B.Cu") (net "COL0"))
 (segment (start 10.9546 19.0019) (end 10.9546 11.5029) (width 0.2) (layer "B.Cu") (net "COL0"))
 (segment (start 10.1951 11.5572) (end 9.6444 11.0065) (width 0.2) (layer "F.Cu") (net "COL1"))
 (segment (start 9.6444 8.0276) (end 9.75 7.922) (width 0.2) (layer "F.Cu") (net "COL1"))
 (segment (start 9.6444 11.0065) (end 9.6444 8.0276) (width 0.2) (layer "F.Cu") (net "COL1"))
 (segment (start 9.75 7.922) (end 9.75 7.1) (width 0.2) (layer "F.Cu") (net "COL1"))
 (via (at 10.1951 11.5572) (size 0.6) (drill 0.3) (layers "F.Cu" "B.Cu") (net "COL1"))
 (segment (start 15.4472 26.8372) (end 15.4472 25.6053) (width 0.2) (layer "B.Cu") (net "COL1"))
 (segment (start 16.62 28.01) (end 15.4472 26.8372) (width 0.2) (layer "B.Cu") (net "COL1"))
 (segment (start 15.4472 25.6053) (end 15.5198 25.5327) (width 0.15) (layer "B.Cu") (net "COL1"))
 (segment (start 15.5198 25.5327) (end 15.5198 24.2441) (width 0.15) (layer "B.Cu") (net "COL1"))
 (segment (start 10.1951 18.9194) (end 10.1951 11.5572) (width 0.2) (layer "B.Cu") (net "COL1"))
 (segment (start 15.5198 24.2441) (end 10.1951 18.9194) (width 0.2) (layer "B.Cu") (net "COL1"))
 (segment (start 13.3246 27.2546) (end 13.3246 4.9227) (width 0.2) (layer "F.Cu") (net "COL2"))
 (segment (start 16.62 30.55) (end 13.3246 27.2546) (width 0.2) (layer "F.Cu") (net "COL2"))
 (segment (start 13.3246 4.9227) (end 12.0436 3.6417) (width 0.2) (layer "F.Cu") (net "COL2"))
 (segment (start 12.0436 3.6417) (end 11.4838 3.6417) (width 0.2) (layer "F.Cu") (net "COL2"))
 (segment (start 11.4838 3.6417) (end 9.25 5.8755) (width 0.2) (layer "F.Cu") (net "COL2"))
 (segment (start 9.25 5.8755) (end 9.25 6.1983) (width 0.2) (layer "F.Cu") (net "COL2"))
 (segment (start 9.25 7.1) (end 9.25 6.1983) (width 0.2) (layer "F.Cu") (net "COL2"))
 (segment (start 12.8401 29.3101) (end 12.8401 14.867) (width 0.2) (layer "F.Cu") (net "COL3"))
 (segment (start 8.75 10.9399) (end 8.75 7.1) (width 0.2) (layer "F.Cu") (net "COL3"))
 (segment (start 12.8401 14.867) (end 12.5169 14.5438) (width 0.2) (layer "F.Cu") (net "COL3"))
 (segment (start 12.5169 14.5438) (end 12.3539 14.5438) (width 0.2) (layer "F.Cu") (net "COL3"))
 (segment (start 16.62 33.09) (end 12.8401 29.3101) (width 0.2) (layer "F.Cu") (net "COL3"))
 (segment (start 12.3539 14.5438) (end 8.75 10.9399) (width 0.2) (layer "F.Cu") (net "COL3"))
 (segment (start 14.5702 8.1058) (end 14.5702 27.0296) (width 0.2) (layer "F.Cu") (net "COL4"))
 (segment (start 12.0015 2.4468) (end 15.6809 2.4468) (width 0.2) (layer "F.Cu") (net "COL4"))
 (segment (start 8.25 6.1983) (end 12.0015 2.4468) (width 0.2) (layer "F.Cu") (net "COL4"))
 (segment (start 15.6809 2.4468) (end 15.8017 2.5676) (width 0.2) (layer "F.Cu") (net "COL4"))
 (segment (start 15.8017 6.8743) (end 14.5702 8.1058) (width 0.2) (layer "F.Cu") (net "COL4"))
 (segment (start 15.8017 2.5676) (end 15.8017 6.8743) (width 0.2) (layer "F.Cu") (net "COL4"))
 (segment (start 8.25 7.1) (end 8.25 6.1983) (width 0.2) (layer "F.Cu") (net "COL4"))
 (via (at 14.5702 27.0296) (size 0.6) (drill 0.3) (layers "F.Cu" "B.Cu") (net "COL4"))
 (segment (start 14.5702 27.0296) (end 14.5702 31.1126) (width 0.2) (layer "B.Cu") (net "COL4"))
 (segment (start 15.4474 32.7067) (end 15.6226 32.5315) (width 0.15) (layer "B.Cu") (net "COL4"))
 (segment (start 15.5198 32.9545) (end 15.4836 32.9183) (width 0.15) (layer "B.Cu") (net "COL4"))
 (segment (start 14.5702 31.1126) (end 15.6226 32.165) (width 0.2) (layer "B.Cu") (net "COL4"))
 (segment (start 16.62 35.63) (end 15.7842 34.7942) (width 0.2) (layer "B.Cu") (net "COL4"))
 (segment (start 15.5198 34.7942) (end 15.5198 32.9545) (width 0.15) (layer "B.Cu") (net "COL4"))
 (segment (start 15.4836 32.9183) (end 15.4474 32.8821) (width 0.2) (layer "B.Cu") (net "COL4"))
 (segment (start 15.6226 32.5315) (end 15.6226 32.165) (width 0.15) (layer "B.Cu") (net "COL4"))
 (segment (start 15.4474 32.8821) (end 15.4474 32.7067) (width 0.2) (layer "B.Cu") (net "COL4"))
 (segment (start 15.7842 34.7942) (end 15.5198 34.7942) (width 0.2) (layer "B.Cu") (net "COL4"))
 (segment (start 13.8252 38.17) (end 4.2152 28.56) (width 0.2) (layer "F.Cu") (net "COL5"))
 (segment (start 7.75 5.8064) (end 7.75 7.1) (width 0.2) (layer "F.Cu") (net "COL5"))
 (segment (start 4.2152 26.9363) (end 4.3818 26.7697) (width 0.2) (layer "F.Cu") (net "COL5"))
 (segment (start 4.2152 28.56) (end 4.2152 26.9363) (width 0.2) (layer "F.Cu") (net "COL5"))
 (segment (start 7.3189 5.3753) (end 7.75 5.8064) (width 0.2) (layer "F.Cu") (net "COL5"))
 (segment (start 4.3818 6.7886) (end 5.7951 5.3753) (width 0.2) (layer "F.Cu") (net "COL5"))
 (segment (start 16.62 38.17) (end 13.8252 38.17) (width 0.2) (layer "F.Cu") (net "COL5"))
 (segment (start 5.7951 5.3753) (end 7.3189 5.3753) (width 0.2) (layer "F.Cu") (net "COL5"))
 (segment (start 4.3818 26.7697) (end 4.3818 6.7886) (width 0.2) (layer "F.Cu") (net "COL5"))
 (segment (start 7.0419 5.9396) (end 7.25 6.1477) (width 0.2) (layer "F.Cu") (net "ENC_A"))
 (segment (start 7.25 6.1477) (end 7.25 7.1) (width 0.2) (layer "F.Cu") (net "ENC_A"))
 (via (at 7.0419 5.9396) (size 0.6) (drill 0.3) (layers "F.Cu" "B.Cu") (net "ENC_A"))
 (segment (start 15.4472 10.7394) (end 13.2833 8.5755) (width 0.15) (layer "B.Cu") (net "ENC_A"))
 (segment (start 15.4472 19.2172) (end 15.4472 17.7239) (width 0.2) (layer "B.Cu") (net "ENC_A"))
 (segment (start 16.62 20.39) (end 15.4472 19.2172) (width 0.2) (layer "B.Cu") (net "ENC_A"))
 (segment (start 12.1985 3.2667) (end 9.7148 3.2667) (width 0.2) (layer "B.Cu") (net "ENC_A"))
 (segment (start 9.7148 3.2667) (end 7.0419 5.9396) (width 0.2) (layer "B.Cu") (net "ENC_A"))
 (segment (start 13.2833 8.5755) (end 13.2833 4.3515) (width 0.2) (layer "B.Cu") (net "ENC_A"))
 (segment (start 13.2833 4.3515) (end 12.1985 3.2667) (width 0.2) (layer "B.Cu") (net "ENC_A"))
 (segment (start 15.4472 17.7239) (end 15.4472 10.7394) (width 0.15) (layer "B.Cu") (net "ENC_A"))
 (segment (start 6.75 7.1) (end 6.75 10.7075) (width 0.2) (layer "F.Cu") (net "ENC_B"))
 (segment (start 6.75 10.7075) (end 11.7132 15.6707) (width 0.2) (layer "F.Cu") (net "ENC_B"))
 (via (at 11.7132 15.6707) (size 0.6) (drill 0.3) (layers "F.Cu" "B.Cu") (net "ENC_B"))
 (segment (start 15.5198 21.044) (end 15.5198 20.4289) (width 0.15) (layer "B.Cu") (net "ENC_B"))
 (segment (start 15.5198 21.8298) (end 15.5198 21.044) (width 0.2) (layer "B.Cu") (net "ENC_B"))
 (segment (start 15.3785 20.2876) (end 11.7132 16.6223) (width 0.2) (layer "B.Cu") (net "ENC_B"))
 (segment (start 11.7132 16.6223) (end 11.7132 15.6707) (width 0.2) (layer "B.Cu") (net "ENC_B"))
 (segment (start 15.5198 20.4289) (end 15.3785 20.2876) (width 0.15) (layer "B.Cu") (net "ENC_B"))
 (segment (start 16.62 22.93) (end 15.5198 21.8298) (width 0.2) (layer "B.Cu") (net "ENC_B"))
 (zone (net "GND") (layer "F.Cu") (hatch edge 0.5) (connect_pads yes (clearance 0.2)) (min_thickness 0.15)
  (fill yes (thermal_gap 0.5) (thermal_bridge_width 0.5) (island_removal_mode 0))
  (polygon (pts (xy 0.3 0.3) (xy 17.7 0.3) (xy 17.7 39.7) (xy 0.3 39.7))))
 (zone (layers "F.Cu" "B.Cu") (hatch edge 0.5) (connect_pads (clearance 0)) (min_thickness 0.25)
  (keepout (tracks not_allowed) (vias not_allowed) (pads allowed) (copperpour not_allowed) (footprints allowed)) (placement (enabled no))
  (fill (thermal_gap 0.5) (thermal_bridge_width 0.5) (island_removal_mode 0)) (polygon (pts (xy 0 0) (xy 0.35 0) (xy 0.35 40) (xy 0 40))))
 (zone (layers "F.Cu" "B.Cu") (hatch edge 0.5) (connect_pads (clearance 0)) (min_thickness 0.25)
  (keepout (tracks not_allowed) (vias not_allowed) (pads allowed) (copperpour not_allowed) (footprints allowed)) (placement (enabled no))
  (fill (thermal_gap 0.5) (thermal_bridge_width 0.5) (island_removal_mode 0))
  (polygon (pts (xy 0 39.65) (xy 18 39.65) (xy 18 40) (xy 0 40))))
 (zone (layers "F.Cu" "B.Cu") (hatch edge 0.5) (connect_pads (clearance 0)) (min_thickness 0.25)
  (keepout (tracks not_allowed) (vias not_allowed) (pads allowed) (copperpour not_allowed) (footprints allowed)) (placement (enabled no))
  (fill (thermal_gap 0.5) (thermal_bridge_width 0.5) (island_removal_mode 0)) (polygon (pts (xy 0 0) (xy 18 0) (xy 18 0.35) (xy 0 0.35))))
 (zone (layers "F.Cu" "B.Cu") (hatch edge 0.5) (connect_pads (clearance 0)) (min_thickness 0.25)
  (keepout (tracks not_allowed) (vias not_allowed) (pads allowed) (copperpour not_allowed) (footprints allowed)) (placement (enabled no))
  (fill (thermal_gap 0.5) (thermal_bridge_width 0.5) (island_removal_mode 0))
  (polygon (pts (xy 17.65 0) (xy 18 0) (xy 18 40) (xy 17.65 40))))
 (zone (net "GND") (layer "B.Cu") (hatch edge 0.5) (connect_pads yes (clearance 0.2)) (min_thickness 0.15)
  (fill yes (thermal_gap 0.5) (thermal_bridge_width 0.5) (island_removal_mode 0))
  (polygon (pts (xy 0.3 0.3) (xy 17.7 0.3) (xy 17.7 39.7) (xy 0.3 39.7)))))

